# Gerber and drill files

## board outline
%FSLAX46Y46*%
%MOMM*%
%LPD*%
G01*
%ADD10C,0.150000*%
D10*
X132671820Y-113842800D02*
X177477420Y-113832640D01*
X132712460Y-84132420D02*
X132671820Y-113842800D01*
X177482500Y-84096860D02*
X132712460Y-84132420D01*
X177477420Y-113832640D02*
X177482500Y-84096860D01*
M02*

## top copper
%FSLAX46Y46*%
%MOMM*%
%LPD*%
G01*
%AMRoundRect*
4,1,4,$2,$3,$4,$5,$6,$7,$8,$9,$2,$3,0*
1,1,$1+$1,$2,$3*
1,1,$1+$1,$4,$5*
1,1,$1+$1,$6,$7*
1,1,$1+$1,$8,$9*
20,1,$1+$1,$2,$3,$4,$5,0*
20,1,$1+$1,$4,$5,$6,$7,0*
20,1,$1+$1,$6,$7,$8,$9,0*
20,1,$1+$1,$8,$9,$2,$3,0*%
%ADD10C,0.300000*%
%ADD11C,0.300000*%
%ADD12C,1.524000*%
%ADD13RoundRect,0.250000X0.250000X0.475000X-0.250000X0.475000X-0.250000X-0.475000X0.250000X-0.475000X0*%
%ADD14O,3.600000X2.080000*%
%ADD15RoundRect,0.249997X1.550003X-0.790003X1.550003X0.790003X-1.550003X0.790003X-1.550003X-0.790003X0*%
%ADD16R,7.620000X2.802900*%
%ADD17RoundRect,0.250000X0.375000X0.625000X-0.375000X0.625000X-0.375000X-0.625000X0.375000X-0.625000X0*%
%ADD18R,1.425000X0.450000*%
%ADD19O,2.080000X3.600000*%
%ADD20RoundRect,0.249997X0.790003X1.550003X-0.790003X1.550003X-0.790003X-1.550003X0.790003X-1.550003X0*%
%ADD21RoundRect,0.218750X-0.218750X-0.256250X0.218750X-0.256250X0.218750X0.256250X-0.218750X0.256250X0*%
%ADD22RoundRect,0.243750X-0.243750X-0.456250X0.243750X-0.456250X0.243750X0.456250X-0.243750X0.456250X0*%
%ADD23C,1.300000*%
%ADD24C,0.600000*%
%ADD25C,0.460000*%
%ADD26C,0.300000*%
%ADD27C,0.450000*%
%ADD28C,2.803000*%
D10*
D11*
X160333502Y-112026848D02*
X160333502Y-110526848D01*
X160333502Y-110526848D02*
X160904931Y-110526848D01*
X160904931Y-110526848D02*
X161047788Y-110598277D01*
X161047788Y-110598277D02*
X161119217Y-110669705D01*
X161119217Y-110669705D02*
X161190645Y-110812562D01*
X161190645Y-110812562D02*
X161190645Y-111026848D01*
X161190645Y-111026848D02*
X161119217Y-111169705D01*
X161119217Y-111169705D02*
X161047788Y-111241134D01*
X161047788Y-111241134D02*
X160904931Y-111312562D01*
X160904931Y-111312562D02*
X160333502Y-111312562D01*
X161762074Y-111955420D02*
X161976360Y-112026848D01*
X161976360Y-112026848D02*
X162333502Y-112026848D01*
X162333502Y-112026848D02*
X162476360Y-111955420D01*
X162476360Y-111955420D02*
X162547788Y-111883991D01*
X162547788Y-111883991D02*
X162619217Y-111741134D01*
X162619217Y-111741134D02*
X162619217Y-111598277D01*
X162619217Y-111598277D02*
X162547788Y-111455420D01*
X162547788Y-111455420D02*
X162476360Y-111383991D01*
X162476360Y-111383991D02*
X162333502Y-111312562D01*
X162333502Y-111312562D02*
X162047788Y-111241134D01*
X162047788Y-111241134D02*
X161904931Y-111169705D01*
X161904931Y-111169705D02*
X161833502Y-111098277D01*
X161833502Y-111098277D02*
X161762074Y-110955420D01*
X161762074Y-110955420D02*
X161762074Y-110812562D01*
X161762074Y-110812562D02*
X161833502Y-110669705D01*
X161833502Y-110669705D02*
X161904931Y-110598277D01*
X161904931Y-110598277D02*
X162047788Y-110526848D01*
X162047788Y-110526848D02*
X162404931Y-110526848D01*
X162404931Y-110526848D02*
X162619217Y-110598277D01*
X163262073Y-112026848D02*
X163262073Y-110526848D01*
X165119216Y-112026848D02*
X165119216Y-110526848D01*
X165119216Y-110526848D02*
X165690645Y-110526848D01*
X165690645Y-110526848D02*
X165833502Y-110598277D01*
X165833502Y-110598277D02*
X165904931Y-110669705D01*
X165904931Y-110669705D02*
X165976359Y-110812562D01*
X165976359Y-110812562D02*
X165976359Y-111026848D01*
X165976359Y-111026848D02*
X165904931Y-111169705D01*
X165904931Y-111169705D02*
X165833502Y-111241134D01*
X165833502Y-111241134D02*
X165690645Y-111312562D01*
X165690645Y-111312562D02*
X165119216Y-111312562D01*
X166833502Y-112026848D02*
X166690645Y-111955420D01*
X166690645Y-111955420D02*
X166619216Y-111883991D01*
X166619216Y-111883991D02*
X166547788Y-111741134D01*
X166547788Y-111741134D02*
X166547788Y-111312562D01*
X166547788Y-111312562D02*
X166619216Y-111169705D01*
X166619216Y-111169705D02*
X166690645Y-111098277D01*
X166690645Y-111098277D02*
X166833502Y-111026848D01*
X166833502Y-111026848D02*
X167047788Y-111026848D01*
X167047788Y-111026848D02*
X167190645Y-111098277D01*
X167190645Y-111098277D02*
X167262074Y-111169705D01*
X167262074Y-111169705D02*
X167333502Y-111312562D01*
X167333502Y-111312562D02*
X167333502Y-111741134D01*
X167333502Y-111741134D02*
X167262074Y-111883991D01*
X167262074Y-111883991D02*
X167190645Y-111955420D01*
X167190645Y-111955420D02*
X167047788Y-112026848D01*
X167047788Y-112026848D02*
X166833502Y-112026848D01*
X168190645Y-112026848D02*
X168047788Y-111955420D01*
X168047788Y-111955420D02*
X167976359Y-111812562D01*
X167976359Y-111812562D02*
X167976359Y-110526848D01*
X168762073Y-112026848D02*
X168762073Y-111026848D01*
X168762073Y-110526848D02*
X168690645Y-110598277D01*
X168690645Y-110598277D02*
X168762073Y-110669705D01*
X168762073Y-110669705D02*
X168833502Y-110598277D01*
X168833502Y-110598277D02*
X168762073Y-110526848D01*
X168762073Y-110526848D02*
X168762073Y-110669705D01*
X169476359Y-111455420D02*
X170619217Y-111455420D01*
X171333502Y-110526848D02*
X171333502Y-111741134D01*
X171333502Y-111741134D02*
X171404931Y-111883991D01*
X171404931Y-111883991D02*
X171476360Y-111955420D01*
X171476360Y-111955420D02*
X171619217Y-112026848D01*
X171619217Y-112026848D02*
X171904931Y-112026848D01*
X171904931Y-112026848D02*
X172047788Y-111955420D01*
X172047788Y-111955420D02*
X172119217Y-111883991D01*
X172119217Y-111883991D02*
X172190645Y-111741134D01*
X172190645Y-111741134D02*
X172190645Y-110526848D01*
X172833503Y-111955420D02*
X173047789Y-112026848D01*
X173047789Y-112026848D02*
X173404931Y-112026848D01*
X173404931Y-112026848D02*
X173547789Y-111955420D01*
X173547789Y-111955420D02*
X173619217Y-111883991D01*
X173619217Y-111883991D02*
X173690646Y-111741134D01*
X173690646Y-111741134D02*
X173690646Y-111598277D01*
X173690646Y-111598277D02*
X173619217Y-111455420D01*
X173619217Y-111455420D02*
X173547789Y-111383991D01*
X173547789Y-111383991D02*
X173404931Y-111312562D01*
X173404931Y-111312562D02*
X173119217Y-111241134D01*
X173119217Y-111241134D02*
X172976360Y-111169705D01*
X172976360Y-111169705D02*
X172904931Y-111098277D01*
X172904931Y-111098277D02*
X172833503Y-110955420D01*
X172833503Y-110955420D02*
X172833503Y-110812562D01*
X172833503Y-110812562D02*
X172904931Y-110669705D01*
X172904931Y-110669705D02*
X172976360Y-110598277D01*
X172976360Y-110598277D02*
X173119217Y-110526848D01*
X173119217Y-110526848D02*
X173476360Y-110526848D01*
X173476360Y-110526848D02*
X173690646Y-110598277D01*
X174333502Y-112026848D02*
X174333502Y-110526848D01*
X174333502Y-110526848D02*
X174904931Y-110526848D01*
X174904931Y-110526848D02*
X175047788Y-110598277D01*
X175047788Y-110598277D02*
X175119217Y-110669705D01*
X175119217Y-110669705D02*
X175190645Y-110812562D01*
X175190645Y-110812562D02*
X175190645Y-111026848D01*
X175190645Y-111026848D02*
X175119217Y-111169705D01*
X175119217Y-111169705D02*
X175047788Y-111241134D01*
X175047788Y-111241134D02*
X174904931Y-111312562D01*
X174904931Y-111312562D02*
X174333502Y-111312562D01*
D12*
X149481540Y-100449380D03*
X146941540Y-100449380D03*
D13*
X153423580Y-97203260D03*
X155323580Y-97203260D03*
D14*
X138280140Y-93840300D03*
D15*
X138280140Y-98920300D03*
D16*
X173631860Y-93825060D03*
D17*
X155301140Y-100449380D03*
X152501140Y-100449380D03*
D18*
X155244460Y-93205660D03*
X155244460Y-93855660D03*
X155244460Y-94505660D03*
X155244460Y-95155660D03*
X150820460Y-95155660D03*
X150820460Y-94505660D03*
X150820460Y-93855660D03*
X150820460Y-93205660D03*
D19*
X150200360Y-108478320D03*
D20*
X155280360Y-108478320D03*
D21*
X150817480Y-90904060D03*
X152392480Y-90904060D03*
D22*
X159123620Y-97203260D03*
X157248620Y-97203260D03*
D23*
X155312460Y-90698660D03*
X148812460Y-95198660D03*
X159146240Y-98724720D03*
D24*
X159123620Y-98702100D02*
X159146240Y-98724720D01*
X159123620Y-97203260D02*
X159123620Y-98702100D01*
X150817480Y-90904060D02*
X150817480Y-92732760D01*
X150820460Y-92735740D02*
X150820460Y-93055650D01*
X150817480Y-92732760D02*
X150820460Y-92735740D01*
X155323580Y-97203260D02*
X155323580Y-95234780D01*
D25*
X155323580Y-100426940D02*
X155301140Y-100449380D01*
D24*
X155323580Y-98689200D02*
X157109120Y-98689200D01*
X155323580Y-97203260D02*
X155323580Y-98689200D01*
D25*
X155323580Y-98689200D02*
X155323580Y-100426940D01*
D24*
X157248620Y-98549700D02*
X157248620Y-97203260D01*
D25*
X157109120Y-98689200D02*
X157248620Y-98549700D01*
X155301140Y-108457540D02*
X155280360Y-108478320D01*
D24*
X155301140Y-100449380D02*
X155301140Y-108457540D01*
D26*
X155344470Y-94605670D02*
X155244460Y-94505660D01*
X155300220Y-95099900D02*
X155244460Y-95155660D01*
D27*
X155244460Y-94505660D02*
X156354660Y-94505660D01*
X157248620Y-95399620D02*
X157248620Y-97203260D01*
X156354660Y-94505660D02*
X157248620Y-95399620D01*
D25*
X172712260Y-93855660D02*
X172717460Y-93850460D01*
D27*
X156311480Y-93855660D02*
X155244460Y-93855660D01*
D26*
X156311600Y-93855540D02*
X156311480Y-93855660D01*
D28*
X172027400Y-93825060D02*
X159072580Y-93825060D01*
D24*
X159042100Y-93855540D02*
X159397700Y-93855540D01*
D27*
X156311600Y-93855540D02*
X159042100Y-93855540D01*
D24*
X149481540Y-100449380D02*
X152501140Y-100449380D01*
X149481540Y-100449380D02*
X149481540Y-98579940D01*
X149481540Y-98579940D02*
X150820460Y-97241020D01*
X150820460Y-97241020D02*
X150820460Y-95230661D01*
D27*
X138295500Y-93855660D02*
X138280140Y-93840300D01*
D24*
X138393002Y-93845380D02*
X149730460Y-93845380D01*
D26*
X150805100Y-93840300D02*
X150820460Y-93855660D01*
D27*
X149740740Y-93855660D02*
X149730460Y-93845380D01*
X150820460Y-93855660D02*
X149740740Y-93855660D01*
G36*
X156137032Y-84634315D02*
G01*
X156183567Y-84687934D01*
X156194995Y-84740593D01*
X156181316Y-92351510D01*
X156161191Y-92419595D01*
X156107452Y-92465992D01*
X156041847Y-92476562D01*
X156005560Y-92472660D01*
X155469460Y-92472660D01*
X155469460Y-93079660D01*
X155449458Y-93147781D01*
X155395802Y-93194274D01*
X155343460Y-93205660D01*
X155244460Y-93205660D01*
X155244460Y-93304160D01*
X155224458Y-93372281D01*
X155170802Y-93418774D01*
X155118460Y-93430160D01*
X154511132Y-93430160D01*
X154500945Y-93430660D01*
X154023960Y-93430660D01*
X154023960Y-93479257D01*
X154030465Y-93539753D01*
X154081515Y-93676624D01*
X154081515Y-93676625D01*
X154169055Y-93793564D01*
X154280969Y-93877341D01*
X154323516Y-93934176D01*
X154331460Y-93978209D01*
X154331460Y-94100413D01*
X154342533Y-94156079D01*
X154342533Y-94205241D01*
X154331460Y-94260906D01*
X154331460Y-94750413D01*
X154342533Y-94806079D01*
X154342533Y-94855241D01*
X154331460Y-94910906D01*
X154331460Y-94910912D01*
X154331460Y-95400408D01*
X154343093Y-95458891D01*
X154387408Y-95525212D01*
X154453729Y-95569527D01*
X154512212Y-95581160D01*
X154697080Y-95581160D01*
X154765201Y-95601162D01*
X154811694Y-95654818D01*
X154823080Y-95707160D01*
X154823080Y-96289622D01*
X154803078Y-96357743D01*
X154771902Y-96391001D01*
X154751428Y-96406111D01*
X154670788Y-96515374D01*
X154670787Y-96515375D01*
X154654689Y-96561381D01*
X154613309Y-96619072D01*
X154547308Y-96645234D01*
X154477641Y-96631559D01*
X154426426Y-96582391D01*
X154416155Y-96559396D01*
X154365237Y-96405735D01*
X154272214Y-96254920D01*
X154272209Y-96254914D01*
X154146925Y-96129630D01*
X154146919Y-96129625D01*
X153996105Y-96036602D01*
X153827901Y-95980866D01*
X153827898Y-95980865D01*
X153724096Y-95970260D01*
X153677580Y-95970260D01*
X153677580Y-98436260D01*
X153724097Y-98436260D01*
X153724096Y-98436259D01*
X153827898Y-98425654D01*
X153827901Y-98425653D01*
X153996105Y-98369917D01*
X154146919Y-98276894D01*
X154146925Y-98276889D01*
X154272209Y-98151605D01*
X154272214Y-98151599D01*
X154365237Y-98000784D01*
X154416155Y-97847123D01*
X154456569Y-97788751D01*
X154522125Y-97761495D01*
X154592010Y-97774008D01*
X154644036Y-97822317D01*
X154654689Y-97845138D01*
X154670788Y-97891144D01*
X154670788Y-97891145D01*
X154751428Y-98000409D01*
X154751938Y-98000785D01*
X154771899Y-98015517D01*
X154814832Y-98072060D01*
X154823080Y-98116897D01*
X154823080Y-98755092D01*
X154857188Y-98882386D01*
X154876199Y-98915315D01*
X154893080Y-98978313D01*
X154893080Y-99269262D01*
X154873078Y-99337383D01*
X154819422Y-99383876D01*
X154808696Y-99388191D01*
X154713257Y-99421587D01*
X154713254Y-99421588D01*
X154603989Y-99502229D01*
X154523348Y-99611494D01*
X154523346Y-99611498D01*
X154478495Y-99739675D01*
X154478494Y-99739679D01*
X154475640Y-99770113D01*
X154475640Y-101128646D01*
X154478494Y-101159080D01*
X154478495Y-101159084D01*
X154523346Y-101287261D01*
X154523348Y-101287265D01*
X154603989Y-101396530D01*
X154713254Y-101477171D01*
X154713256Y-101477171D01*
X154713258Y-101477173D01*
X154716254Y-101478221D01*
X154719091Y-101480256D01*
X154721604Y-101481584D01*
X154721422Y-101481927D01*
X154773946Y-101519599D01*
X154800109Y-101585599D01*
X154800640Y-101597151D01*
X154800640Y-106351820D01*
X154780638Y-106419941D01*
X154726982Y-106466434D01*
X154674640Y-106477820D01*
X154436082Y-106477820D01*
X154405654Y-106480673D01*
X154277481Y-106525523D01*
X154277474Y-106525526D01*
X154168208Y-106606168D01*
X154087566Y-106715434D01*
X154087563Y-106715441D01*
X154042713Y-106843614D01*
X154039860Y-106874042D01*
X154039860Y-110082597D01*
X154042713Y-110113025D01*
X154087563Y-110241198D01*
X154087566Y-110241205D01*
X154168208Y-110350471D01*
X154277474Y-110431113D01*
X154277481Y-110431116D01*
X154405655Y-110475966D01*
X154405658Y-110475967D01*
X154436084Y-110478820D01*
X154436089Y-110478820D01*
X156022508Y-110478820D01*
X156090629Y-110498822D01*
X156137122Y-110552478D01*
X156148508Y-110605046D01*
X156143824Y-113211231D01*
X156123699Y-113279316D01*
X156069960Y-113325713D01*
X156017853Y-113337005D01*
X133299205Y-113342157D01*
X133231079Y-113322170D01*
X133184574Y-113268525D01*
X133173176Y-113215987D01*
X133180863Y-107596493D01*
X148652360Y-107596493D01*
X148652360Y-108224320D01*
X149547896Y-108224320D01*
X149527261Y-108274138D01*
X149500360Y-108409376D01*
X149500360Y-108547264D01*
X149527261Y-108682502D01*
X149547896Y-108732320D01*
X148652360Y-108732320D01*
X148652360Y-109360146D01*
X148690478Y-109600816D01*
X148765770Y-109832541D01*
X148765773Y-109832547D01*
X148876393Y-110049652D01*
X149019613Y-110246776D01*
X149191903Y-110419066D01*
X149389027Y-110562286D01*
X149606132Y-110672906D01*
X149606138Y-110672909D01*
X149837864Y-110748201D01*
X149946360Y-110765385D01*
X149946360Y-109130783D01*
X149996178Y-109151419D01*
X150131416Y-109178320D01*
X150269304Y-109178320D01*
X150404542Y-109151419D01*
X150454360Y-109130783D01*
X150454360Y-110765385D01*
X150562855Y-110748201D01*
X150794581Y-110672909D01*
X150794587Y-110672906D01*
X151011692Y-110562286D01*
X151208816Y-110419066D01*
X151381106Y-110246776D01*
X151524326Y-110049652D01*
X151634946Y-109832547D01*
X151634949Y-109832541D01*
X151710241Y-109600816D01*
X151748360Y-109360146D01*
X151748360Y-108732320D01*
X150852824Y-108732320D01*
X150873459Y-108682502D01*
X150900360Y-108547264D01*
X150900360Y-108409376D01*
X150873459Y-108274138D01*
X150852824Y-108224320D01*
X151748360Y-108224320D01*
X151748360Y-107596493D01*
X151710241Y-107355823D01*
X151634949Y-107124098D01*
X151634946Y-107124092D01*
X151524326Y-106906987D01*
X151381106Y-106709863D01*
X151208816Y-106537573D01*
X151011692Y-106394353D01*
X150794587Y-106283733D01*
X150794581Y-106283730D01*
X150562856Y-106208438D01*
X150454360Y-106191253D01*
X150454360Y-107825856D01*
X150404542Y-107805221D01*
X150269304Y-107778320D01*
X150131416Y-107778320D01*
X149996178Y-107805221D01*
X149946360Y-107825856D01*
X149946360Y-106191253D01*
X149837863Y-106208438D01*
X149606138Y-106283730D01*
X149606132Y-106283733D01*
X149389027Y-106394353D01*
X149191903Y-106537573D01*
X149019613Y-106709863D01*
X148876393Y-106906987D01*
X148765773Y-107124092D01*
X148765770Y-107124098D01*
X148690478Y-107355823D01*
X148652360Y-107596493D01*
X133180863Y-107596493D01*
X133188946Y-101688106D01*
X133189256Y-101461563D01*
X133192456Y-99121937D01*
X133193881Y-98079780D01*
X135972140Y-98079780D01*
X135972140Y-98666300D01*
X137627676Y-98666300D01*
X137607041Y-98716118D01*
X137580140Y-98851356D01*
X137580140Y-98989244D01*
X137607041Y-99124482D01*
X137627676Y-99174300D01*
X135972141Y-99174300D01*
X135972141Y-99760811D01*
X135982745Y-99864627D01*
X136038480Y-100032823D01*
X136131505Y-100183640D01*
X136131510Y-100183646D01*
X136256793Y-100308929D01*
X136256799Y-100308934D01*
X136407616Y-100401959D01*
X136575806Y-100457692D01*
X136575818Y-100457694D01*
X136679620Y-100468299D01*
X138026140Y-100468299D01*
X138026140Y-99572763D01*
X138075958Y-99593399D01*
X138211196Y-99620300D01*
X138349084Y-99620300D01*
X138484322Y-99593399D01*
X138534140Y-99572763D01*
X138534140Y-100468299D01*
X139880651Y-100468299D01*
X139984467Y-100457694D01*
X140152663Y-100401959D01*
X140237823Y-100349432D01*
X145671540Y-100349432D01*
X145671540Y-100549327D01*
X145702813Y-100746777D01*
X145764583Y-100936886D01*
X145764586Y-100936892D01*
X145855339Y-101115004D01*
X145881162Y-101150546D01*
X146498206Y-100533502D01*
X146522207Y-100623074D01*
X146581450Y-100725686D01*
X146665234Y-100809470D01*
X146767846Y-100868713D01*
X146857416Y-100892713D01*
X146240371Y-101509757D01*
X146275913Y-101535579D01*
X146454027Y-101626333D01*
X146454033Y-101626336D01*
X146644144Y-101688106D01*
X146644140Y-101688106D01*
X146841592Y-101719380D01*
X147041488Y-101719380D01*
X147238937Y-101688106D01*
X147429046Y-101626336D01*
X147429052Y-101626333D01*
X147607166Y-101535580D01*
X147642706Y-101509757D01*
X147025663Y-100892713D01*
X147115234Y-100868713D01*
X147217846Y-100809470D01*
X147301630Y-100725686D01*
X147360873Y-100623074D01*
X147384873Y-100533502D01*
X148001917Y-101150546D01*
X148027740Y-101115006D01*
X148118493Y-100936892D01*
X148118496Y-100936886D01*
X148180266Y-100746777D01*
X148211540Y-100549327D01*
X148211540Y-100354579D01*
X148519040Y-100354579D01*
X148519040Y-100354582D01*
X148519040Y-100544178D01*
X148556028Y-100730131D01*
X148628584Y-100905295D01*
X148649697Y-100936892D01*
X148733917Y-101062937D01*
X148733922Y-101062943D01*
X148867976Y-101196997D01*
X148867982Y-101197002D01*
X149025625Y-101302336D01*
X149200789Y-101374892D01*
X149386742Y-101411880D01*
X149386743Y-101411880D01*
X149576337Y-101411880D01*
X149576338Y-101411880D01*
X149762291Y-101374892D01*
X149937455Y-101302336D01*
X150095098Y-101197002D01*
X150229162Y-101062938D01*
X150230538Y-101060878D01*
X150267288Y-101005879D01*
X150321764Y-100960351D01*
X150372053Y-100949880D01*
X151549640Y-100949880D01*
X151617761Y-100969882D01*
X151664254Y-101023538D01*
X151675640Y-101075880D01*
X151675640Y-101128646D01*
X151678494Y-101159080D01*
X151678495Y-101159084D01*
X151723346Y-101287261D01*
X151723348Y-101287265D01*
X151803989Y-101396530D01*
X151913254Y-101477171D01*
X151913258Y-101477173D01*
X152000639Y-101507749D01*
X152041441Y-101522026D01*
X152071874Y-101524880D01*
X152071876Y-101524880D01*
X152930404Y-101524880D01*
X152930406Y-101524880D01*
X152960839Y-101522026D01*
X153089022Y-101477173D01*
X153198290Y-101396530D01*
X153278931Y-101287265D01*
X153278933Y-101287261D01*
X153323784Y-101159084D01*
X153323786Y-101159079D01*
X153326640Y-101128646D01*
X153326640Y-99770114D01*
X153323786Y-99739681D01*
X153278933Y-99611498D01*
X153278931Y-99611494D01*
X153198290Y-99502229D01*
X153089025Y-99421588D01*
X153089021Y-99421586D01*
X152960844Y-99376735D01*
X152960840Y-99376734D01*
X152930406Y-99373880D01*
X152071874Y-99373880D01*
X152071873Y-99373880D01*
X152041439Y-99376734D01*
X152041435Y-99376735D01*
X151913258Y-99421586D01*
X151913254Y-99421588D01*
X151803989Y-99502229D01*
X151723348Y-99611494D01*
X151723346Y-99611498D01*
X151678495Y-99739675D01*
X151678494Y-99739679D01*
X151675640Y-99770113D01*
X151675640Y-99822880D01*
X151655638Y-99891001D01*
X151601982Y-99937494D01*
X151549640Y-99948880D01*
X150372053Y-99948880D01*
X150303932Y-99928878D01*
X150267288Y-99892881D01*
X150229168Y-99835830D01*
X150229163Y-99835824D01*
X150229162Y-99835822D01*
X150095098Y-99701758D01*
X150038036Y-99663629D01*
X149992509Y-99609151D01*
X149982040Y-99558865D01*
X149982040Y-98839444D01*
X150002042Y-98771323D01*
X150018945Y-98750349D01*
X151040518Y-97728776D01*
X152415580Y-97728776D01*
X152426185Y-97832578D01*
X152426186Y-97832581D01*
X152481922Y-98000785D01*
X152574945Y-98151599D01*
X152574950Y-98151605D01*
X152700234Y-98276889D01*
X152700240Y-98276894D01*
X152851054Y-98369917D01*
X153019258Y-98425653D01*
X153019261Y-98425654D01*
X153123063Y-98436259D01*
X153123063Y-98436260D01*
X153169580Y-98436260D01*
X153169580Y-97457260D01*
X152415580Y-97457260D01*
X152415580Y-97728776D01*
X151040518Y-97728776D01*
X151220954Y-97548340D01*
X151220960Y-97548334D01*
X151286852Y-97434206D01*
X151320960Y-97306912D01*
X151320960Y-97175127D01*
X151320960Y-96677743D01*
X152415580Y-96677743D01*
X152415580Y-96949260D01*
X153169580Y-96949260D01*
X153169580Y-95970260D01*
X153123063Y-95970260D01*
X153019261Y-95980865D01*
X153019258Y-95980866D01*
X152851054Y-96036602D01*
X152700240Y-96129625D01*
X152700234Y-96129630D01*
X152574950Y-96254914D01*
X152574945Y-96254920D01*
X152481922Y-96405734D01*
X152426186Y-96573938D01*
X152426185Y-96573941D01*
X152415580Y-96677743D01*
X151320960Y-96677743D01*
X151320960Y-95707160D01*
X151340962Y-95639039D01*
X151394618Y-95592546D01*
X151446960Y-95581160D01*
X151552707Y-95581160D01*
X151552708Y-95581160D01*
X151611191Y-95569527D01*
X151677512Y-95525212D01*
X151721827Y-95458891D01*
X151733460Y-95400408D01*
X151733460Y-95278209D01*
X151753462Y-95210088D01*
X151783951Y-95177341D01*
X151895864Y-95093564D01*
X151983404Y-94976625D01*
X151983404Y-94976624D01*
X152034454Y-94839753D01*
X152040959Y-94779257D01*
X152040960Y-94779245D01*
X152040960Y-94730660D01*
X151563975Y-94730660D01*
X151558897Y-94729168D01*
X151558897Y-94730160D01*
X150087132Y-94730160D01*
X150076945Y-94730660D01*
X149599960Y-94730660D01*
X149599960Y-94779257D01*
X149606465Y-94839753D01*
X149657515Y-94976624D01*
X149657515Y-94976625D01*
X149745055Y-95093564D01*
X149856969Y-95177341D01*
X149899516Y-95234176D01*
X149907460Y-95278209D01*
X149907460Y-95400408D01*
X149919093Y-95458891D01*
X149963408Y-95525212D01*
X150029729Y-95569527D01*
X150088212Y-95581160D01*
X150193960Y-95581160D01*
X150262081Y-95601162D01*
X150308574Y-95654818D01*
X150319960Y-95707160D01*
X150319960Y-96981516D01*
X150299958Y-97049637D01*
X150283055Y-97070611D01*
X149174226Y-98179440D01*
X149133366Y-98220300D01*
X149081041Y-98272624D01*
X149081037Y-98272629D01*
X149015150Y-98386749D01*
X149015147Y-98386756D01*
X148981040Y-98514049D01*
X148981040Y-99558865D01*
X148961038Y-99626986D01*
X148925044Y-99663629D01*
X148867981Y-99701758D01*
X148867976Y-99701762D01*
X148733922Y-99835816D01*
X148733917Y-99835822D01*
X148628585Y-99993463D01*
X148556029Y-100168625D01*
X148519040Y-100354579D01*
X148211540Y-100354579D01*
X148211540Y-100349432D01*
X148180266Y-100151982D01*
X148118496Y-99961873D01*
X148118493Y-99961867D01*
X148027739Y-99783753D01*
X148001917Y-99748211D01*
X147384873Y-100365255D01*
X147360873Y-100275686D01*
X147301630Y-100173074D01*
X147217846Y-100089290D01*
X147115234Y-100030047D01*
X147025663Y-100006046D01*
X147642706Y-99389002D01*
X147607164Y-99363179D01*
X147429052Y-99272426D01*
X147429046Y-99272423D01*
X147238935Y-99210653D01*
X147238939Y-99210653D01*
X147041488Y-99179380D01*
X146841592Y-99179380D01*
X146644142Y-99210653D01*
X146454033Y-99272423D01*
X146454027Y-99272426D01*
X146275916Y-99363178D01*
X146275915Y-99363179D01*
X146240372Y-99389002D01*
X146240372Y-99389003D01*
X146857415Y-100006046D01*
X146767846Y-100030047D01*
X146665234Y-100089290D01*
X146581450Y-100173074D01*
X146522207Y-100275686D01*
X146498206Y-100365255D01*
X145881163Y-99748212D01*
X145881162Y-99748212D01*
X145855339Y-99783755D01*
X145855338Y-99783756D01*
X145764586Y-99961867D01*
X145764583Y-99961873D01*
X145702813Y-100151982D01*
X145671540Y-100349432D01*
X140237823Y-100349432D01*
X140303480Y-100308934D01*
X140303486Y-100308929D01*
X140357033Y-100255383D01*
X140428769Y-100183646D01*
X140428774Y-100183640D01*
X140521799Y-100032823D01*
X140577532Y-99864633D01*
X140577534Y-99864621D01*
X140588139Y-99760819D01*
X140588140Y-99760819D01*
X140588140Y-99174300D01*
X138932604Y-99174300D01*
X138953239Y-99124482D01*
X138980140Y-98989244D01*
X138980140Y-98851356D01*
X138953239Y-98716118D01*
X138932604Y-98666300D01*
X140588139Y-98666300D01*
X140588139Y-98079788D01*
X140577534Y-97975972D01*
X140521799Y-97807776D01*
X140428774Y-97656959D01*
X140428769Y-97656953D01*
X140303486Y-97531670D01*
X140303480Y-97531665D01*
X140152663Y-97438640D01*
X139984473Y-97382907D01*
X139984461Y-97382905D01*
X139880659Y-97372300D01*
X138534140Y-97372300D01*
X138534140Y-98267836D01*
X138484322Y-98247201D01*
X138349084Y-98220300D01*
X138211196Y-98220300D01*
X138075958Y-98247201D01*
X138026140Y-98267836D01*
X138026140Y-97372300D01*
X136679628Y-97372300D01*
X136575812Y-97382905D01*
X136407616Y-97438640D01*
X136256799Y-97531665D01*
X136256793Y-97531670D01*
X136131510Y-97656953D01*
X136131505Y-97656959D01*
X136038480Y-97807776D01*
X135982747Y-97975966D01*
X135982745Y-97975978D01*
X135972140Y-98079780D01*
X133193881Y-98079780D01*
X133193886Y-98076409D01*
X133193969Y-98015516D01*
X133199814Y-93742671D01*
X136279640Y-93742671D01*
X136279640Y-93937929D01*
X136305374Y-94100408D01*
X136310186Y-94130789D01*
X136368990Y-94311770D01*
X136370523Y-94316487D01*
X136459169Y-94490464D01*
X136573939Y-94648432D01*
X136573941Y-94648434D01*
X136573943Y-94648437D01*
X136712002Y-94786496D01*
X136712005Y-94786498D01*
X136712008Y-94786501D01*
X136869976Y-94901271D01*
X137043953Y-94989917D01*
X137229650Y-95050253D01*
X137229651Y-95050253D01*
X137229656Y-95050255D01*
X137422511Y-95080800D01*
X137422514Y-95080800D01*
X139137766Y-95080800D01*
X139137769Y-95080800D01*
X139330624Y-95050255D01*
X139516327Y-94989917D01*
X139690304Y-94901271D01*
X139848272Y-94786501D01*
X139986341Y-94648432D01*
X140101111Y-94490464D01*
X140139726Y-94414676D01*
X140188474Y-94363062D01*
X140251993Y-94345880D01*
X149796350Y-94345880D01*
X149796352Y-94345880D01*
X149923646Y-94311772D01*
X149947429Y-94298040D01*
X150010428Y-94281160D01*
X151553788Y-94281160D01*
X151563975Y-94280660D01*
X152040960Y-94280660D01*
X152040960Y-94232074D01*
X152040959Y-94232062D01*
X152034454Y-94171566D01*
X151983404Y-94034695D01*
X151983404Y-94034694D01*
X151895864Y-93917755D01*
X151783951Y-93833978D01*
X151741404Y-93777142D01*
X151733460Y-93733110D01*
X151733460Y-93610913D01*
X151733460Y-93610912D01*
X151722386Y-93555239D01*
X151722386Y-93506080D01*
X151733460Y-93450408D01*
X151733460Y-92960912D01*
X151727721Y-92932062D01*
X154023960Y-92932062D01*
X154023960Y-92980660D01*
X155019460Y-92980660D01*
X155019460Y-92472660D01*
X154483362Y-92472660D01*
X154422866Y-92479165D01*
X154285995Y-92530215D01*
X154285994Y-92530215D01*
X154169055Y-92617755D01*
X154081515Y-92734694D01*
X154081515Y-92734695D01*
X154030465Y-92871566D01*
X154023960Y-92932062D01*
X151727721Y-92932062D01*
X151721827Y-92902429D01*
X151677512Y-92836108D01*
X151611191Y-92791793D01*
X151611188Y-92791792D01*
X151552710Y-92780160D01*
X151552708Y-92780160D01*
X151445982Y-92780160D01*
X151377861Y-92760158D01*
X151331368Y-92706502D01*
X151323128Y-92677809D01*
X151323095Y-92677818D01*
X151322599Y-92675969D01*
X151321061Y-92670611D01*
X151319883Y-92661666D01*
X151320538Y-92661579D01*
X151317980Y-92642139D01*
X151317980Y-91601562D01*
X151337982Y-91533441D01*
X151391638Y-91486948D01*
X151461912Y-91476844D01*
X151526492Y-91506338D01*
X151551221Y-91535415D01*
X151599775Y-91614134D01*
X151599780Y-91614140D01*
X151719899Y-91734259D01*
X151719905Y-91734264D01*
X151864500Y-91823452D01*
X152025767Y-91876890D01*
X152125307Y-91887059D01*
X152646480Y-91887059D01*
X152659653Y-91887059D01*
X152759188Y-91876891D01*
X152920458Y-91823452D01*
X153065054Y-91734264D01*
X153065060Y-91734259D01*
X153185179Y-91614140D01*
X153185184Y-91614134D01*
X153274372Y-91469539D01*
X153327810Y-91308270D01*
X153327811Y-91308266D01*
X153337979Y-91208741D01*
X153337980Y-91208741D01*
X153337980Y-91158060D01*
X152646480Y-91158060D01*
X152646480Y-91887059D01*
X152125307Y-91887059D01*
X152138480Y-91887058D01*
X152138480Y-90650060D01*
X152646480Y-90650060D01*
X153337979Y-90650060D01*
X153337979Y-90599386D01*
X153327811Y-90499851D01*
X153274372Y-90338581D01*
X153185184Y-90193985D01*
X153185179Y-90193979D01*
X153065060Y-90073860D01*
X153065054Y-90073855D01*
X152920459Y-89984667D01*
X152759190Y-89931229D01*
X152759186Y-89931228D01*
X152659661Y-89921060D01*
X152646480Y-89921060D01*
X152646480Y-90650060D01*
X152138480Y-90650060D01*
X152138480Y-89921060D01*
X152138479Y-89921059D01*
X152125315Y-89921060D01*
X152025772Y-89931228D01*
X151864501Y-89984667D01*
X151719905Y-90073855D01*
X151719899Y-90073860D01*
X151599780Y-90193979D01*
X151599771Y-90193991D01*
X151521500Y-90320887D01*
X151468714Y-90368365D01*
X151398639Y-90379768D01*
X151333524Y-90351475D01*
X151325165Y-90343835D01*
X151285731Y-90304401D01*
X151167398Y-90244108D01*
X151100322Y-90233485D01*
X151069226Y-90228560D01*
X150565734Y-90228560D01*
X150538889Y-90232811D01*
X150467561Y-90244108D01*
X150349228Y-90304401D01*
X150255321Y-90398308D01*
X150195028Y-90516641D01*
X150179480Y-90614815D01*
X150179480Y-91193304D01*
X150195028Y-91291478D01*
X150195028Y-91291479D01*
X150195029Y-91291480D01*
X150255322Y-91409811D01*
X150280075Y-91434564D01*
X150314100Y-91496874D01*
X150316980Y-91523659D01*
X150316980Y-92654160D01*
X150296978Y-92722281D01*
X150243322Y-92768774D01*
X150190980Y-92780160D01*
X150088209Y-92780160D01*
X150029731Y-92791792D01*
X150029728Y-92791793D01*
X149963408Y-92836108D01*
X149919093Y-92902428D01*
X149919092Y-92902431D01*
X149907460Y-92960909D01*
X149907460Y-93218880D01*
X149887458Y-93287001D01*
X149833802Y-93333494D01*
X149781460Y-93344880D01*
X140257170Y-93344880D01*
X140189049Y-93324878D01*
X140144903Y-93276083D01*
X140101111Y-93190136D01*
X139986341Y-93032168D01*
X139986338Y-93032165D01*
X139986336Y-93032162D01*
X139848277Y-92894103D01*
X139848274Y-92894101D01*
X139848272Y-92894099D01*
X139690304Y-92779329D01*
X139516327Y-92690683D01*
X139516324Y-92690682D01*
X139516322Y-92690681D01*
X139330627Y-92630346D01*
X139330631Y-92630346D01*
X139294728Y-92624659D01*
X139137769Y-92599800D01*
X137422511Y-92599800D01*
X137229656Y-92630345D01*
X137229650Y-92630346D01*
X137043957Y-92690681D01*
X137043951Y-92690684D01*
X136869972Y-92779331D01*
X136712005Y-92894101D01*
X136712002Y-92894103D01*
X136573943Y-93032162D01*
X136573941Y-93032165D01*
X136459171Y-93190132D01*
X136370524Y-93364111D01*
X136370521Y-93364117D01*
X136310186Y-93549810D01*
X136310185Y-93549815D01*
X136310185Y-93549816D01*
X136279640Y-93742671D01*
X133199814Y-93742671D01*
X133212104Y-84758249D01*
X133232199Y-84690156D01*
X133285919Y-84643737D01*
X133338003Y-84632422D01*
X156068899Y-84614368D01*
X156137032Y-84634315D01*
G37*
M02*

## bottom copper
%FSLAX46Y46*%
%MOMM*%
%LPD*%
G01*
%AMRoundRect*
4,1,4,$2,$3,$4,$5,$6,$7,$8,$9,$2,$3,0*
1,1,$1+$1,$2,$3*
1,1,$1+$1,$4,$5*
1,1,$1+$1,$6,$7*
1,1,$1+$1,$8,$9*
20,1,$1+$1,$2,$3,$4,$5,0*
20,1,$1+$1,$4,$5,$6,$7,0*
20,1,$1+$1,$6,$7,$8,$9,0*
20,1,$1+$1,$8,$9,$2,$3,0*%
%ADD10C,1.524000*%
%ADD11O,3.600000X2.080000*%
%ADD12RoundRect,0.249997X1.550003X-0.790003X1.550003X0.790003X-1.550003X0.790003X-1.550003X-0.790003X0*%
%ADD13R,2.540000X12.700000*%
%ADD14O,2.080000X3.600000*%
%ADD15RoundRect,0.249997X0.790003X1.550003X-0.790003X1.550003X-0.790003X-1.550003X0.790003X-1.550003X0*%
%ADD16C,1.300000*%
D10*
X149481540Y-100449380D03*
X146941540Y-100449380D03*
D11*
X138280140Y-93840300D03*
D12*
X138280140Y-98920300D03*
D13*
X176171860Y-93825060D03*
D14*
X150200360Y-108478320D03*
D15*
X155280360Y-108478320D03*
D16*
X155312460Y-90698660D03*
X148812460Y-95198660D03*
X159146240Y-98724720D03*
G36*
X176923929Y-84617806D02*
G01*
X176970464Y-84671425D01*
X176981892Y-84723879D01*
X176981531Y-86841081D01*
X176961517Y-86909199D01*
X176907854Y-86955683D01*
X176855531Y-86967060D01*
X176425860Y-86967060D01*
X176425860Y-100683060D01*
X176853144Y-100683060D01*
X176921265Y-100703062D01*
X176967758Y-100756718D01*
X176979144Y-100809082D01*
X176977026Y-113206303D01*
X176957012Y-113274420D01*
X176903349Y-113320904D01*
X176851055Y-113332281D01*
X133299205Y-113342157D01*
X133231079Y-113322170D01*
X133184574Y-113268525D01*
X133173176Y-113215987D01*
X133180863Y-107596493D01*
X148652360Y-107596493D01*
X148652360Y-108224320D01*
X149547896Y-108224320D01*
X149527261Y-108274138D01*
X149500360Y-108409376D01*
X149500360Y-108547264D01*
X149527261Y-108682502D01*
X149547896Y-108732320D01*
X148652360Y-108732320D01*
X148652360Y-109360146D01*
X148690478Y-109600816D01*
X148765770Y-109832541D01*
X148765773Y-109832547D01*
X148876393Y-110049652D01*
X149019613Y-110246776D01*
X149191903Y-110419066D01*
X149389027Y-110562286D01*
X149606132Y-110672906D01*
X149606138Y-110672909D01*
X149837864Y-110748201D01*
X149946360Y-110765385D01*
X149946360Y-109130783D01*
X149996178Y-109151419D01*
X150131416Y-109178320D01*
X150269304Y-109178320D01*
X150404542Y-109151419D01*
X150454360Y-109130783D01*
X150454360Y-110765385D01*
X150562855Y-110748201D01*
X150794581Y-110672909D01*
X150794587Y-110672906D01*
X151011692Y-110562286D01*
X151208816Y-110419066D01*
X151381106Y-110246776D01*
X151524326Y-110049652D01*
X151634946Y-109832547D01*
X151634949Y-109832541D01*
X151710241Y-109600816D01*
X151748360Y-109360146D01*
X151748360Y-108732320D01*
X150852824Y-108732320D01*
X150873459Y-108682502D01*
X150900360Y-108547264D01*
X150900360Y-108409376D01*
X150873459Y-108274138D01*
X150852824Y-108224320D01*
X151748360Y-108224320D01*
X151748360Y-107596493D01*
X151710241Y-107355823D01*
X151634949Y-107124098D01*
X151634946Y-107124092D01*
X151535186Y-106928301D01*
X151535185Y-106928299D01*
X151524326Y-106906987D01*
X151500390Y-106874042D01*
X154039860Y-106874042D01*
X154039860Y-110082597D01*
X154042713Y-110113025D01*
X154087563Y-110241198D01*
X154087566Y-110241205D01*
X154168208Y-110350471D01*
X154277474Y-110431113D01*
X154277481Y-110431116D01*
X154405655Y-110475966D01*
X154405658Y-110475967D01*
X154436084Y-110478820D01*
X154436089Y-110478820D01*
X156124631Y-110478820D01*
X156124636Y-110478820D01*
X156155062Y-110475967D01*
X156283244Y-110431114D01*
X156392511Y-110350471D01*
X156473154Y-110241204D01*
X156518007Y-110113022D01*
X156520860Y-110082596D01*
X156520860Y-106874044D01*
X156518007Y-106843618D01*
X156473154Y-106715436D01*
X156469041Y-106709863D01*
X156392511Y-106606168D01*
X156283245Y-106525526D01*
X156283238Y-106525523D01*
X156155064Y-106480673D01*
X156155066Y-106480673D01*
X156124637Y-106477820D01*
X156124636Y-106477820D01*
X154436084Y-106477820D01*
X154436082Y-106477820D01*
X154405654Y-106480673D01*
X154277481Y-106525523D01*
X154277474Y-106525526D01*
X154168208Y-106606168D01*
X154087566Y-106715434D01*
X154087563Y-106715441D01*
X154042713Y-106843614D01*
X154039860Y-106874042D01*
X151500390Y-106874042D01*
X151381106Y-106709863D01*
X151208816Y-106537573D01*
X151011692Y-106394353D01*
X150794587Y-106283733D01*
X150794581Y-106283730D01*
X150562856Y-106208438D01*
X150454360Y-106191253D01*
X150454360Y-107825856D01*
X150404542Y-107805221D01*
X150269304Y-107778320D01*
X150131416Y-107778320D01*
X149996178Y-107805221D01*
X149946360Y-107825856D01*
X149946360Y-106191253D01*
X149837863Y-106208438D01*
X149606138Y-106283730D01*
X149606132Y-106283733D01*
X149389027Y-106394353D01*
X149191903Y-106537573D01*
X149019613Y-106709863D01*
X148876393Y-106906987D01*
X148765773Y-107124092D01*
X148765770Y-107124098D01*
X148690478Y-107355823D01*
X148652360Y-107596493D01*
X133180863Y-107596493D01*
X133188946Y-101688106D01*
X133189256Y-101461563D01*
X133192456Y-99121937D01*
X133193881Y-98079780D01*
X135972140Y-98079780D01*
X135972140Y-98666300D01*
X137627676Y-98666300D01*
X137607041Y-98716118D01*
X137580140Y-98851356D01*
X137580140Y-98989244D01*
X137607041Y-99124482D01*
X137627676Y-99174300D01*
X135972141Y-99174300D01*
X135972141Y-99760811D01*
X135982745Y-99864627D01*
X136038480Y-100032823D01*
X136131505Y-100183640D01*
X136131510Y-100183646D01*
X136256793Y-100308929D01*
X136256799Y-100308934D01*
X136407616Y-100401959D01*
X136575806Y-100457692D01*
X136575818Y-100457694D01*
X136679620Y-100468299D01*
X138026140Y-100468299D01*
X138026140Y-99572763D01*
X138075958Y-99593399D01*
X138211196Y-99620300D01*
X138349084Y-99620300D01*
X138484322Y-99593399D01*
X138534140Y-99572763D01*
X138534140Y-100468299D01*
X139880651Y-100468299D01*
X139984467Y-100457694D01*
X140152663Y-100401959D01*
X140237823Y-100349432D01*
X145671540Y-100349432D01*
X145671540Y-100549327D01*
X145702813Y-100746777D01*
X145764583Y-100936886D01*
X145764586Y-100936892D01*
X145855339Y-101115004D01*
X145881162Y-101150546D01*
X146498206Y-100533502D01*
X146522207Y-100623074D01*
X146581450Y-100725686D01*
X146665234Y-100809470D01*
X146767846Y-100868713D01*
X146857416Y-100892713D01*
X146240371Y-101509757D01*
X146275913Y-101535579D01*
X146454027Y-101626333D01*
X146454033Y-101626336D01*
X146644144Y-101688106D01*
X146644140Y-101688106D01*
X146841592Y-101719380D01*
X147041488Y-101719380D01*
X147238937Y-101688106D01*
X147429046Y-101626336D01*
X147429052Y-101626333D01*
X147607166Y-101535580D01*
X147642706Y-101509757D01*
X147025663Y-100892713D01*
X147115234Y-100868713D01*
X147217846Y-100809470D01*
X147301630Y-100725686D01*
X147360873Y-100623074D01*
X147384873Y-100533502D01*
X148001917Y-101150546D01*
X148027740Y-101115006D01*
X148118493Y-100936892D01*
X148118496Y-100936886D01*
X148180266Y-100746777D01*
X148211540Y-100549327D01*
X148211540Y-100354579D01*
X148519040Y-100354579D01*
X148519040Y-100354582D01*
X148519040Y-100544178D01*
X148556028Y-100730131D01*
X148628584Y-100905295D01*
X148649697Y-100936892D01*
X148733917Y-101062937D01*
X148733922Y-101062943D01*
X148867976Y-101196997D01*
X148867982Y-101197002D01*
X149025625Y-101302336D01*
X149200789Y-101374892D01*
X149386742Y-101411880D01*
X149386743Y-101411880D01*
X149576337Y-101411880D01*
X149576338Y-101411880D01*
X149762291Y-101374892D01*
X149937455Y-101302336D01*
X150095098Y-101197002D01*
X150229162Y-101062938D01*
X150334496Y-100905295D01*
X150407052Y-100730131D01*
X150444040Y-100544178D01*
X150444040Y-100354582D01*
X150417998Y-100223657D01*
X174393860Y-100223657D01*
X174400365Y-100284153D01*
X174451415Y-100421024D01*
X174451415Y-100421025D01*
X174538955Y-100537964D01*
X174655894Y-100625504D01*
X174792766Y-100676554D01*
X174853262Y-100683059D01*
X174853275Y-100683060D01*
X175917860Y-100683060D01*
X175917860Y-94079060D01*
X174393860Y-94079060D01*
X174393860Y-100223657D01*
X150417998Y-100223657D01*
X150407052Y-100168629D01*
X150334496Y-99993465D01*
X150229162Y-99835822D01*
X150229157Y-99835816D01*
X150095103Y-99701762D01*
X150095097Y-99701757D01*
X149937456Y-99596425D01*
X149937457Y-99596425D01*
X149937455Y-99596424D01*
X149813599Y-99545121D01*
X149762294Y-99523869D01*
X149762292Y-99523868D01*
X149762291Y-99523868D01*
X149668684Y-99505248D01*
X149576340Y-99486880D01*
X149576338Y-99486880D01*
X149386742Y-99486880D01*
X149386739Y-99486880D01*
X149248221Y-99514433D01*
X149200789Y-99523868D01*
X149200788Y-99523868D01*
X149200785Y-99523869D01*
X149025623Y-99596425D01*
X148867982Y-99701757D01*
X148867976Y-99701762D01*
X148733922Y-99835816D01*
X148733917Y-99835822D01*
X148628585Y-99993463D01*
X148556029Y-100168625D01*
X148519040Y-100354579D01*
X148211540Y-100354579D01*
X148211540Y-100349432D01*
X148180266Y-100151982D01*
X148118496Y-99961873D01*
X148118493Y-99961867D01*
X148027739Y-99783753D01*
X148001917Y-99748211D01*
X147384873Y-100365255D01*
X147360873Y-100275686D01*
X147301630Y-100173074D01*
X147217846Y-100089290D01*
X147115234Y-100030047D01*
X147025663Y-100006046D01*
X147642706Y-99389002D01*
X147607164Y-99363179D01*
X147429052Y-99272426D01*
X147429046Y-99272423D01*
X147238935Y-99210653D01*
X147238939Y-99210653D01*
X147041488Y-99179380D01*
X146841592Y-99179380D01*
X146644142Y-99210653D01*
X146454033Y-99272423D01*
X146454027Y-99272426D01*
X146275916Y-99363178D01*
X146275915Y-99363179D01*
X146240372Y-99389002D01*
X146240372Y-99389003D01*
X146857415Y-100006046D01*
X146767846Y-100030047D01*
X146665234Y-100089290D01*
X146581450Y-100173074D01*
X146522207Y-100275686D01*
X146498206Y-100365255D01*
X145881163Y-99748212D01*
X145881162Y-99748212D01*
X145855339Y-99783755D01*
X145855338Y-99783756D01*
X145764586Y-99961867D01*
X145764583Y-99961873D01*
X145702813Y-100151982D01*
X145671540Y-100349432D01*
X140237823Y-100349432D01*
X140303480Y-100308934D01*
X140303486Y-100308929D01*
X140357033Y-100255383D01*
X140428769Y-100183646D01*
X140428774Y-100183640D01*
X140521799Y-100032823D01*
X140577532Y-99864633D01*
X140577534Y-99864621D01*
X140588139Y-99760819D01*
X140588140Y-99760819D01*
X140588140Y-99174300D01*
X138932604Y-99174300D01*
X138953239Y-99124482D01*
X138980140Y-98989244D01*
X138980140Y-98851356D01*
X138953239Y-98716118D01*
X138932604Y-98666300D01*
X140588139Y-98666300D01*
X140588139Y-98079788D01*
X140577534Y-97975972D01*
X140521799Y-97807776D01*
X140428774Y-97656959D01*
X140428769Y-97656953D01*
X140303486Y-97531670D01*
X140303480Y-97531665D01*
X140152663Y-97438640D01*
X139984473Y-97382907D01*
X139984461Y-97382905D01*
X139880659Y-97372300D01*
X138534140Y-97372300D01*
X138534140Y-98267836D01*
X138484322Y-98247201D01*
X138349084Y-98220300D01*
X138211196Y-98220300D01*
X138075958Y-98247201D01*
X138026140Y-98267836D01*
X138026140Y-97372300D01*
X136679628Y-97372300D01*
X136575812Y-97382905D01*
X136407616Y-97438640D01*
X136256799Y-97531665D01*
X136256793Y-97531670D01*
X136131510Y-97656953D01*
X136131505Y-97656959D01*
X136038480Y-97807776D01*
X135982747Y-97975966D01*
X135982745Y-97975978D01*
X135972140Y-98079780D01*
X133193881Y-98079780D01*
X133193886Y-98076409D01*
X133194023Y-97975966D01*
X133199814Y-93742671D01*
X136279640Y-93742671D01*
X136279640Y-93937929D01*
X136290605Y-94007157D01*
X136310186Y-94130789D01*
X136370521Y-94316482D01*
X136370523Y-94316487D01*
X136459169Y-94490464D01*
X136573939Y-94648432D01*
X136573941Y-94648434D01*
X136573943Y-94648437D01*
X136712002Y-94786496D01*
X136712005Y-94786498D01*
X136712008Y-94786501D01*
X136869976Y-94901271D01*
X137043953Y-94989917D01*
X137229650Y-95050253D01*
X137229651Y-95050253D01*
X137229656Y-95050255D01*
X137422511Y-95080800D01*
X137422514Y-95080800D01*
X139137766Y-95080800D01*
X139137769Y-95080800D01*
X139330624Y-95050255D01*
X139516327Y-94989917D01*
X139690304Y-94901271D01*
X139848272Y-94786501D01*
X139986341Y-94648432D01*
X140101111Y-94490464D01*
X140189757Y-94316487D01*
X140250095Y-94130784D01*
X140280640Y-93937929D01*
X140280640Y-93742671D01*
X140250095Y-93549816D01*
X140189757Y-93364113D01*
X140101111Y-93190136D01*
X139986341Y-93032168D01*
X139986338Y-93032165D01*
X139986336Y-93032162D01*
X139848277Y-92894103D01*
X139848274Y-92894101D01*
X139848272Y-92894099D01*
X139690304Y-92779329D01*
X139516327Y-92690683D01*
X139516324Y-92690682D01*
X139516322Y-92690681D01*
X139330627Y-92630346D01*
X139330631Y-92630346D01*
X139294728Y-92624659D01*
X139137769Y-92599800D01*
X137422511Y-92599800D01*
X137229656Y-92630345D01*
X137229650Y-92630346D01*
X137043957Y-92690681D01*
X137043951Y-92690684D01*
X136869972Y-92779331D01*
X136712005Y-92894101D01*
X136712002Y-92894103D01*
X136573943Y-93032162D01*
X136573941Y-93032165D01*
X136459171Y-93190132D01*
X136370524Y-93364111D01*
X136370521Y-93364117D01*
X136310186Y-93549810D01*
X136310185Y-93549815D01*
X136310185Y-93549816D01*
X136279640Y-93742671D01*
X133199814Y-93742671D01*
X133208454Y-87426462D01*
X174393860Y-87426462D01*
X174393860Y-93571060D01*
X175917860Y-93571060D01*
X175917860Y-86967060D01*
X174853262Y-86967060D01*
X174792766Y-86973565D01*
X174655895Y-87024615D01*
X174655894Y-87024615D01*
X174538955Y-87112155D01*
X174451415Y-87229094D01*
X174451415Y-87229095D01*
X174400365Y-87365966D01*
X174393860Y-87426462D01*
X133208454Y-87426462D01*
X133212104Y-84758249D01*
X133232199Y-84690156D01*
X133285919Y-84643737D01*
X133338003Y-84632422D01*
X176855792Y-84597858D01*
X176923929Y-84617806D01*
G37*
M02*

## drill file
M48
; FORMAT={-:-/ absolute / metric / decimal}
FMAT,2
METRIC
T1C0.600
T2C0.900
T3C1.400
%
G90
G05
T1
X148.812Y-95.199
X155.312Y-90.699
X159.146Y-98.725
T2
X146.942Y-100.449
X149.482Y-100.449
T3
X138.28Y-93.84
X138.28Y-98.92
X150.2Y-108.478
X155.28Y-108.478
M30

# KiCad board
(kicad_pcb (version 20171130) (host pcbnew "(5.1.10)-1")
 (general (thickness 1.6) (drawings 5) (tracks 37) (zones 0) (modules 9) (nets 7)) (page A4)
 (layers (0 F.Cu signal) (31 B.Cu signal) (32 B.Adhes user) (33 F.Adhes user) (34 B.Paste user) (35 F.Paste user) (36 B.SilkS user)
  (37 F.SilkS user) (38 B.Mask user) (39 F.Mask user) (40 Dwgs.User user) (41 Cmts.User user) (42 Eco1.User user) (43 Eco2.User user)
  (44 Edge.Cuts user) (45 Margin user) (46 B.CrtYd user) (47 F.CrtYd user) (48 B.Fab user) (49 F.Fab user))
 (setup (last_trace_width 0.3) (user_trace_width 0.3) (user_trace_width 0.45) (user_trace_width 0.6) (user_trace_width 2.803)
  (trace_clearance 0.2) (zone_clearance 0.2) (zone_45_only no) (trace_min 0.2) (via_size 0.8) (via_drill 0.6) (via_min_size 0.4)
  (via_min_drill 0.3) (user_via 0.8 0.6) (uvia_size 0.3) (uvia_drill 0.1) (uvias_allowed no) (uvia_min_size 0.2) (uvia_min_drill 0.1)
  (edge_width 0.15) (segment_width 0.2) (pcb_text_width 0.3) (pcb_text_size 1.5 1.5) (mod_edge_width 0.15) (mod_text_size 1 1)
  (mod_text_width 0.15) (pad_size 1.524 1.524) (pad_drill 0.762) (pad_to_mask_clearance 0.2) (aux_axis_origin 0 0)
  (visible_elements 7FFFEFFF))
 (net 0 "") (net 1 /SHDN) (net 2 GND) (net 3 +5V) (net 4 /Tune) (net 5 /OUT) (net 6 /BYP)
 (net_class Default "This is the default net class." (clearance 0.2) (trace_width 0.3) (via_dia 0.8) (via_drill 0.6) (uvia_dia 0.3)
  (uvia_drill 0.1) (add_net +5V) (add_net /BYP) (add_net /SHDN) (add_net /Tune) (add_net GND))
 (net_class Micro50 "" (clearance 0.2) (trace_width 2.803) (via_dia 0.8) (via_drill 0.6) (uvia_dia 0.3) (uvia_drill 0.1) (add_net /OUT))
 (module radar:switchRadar (layer F.Cu) (at 146.94154 100.44938)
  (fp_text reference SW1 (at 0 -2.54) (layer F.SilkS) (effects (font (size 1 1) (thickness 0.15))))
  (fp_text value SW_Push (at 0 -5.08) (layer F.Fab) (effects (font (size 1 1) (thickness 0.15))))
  (pad 2 thru_hole circle (at 2.54 0) (size 1.524 1.524) (drill 0.9) (layers *.Cu *.Mask) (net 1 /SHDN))
  (pad 1 thru_hole circle (at 0 0) (size 1.524 1.524) (drill 0.9) (layers *.Cu *.Mask) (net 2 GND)))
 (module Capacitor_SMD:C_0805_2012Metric (layer F.Cu) (at 154.37358 97.20326 180)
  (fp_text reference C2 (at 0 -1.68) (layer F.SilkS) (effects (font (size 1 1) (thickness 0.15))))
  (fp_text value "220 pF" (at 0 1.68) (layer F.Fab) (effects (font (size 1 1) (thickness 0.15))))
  (pad 2 smd roundrect (at 0.95 0 180) (size 1 1.45) (layers F.Cu F.Paste F.Mask) (roundrect_rratio 0.25) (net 2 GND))
  (pad 1 smd roundrect (at -0.95 0 180) (size 1 1.45) (layers F.Cu F.Paste F.Mask) (roundrect_rratio 0.25) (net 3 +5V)))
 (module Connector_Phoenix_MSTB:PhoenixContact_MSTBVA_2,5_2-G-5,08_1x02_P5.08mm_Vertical (layer F.Cu) (at 138.28014 98.9203 90)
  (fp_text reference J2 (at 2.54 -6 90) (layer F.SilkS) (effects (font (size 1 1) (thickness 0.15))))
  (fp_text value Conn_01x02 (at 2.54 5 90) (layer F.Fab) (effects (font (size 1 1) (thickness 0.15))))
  (pad 2 thru_hole oval (at 5.08 0 90) (size 2.08 3.6) (drill 1.4) (layers *.Cu *.Mask) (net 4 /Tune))
  (pad 1 thru_hole roundrect (at 0 0 90) (size 2.08 3.6) (drill 1.4) (layers *.Cu *.Mask) (roundrect_rratio 0.1201908653846154) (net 2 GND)))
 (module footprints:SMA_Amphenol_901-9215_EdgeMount (layer F.Cu) (at 172.36186 93.82506)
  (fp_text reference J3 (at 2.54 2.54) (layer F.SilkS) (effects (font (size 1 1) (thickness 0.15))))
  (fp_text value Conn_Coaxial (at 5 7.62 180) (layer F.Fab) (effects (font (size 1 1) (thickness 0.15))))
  (pad 1 smd rect (at 1.27 0 90) (size 2.8029 7.62) (layers F.Cu F.Paste F.Mask) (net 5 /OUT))
  (pad 2 smd rect (at 3.81 0 180) (size 2.54 12.7) (layers B.Cu B.Paste B.Mask) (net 2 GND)))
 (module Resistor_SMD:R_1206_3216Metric (layer F.Cu) (at 153.90114 100.44938 180)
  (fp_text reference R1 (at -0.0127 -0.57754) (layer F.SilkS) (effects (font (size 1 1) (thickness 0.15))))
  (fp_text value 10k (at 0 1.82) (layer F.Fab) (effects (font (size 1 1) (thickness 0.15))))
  (pad 1 smd roundrect (at -1.4 0 180) (size 1.25 1.75) (layers F.Cu F.Paste F.Mask) (roundrect_rratio 0.2) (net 3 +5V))
  (pad 2 smd roundrect (at 1.4 0 180) (size 1.25 1.75) (layers F.Cu F.Paste F.Mask) (roundrect_rratio 0.2) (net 1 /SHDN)))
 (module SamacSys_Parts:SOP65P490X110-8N (layer F.Cu) (at 153.03246 94.18066)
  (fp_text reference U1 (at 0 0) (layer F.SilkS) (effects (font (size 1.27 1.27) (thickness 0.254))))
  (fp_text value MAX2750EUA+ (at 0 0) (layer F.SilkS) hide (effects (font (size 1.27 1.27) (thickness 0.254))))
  (pad 8 smd rect (at 2.212 -0.975 90) (size 0.45 1.425) (layers F.Cu F.Paste F.Mask) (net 2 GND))
  (pad 7 smd rect (at 2.212 -0.325 90) (size 0.45 1.425) (layers F.Cu F.Paste F.Mask) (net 5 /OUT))
  (pad 6 smd rect (at 2.212 0.325 90) (size 0.45 1.425) (layers F.Cu F.Paste F.Mask) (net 3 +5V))
  (pad 5 smd rect (at 2.212 0.975 90) (size 0.45 1.425) (layers F.Cu F.Paste F.Mask) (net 3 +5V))
  (pad 4 smd rect (at -2.212 0.975 90) (size 0.45 1.425) (layers F.Cu F.Paste F.Mask) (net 1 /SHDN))
  (pad 3 smd rect (at -2.212 0.325 90) (size 0.45 1.425) (layers F.Cu F.Paste F.Mask) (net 2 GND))
  (pad 2 smd rect (at -2.212 -0.325 90) (size 0.45 1.425) (layers F.Cu F.Paste F.Mask) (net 4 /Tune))
  (pad 1 smd rect (at -2.212 -0.975 90) (size 0.45 1.425) (layers F.Cu F.Paste F.Mask) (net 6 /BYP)))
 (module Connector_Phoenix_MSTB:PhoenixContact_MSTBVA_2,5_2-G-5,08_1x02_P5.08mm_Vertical (layer F.Cu) (at 155.28036 108.47832 180)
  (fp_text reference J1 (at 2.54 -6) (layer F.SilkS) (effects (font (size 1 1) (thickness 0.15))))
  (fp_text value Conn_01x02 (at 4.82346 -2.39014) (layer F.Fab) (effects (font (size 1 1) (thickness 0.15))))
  (pad 2 thru_hole oval (at 5.08 0 180) (size 2.08 3.6) (drill 1.4) (layers *.Cu *.Mask) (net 2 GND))
  (pad 1 thru_hole roundrect (at 0 0 180) (size 2.08 3.6) (drill 1.4) (layers *.Cu *.Mask) (roundrect_rratio 0.1201908653846154) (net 3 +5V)))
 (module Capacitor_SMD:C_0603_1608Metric (layer F.Cu) (at 151.60498 90.90406)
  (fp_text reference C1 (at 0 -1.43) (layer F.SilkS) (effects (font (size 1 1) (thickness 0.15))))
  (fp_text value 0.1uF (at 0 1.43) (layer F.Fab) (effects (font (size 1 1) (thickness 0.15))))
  (pad 1 smd roundrect (at -0.7875 0) (size 0.875 0.95) (layers F.Cu F.Paste F.Mask) (roundrect_rratio 0.25) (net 6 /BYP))
  (pad 2 smd roundrect (at 0.7875 0) (size 0.875 0.95) (layers F.Cu F.Paste F.Mask) (roundrect_rratio 0.25) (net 2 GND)))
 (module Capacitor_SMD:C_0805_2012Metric (layer F.Cu) (at 158.18612 97.20326)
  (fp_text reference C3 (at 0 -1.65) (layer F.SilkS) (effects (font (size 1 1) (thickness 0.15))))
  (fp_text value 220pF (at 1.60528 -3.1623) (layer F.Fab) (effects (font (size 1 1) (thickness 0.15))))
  (pad 2 smd roundrect (at 0.9375 0) (size 0.975 1.4) (layers F.Cu F.Paste F.Mask) (roundrect_rratio 0.25) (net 2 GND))
  (pad 1 smd roundrect (at -0.9375 0) (size 0.975 1.4) (layers F.Cu F.Paste F.Mask) (roundrect_rratio 0.25) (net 3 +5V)))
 (gr_line (start 132.67182 113.8428) (end 177.47742 113.83264) (layer Edge.Cuts) (width 0.15))
 (gr_line (start 132.71246 84.13242) (end 132.67182 113.8428) (layer Edge.Cuts) (width 0.15))
 (gr_line (start 177.4825 84.09686) (end 132.71246 84.13242) (layer Edge.Cuts) (width 0.15))
 (gr_line (start 177.47742 113.83264) (end 177.4825 84.09686) (layer Edge.Cuts) (width 0.15))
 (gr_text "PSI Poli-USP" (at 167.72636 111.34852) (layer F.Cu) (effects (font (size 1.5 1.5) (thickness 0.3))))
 (via (at 155.31246 90.69866) (size 1.3) (drill 0.6) (layers F.Cu B.Cu) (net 2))
 (via (at 148.81246 95.19866) (size 1.3) (drill 0.6) (layers F.Cu B.Cu) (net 2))
 (via (at 159.14624 98.72472) (size 1.3) (drill 0.6) (layers F.Cu B.Cu) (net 2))
 (segment (start 159.12362 98.7021) (end 159.14624 98.72472) (width 0.6) (layer F.Cu) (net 2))
 (segment (start 159.12362 97.20326) (end 159.12362 98.7021) (width 0.6) (layer F.Cu) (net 2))
 (segment (start 150.81748 90.90406) (end 150.81748 92.73276) (width 0.6) (layer F.Cu) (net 6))
 (segment (start 150.82046 92.73574) (end 150.82046 93.05565) (width 0.6) (layer F.Cu) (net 6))
 (segment (start 150.81748 92.73276) (end 150.82046 92.73574) (width 0.6) (layer F.Cu) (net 6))
 (segment (start 155.32358 97.20326) (end 155.32358 95.23478) (width 0.6) (layer F.Cu) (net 3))
 (segment (start 155.32358 100.42694) (end 155.30114 100.44938) (width 0.46) (layer F.Cu) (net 3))
 (segment (start 155.32358 98.6892) (end 157.10912 98.6892) (width 0.6) (layer F.Cu) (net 3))
 (segment (start 155.32358 97.20326) (end 155.32358 98.6892) (width 0.6) (layer F.Cu) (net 3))
 (segment (start 155.32358 98.6892) (end 155.32358 100.42694) (width 0.46) (layer F.Cu) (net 3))
 (segment (start 157.24862 98.5497) (end 157.24862 97.20326) (width 0.6) (layer F.Cu) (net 3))
 (segment (start 157.10912 98.6892) (end 157.24862 98.5497) (width 0.46) (layer F.Cu) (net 3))
 (segment (start 155.30114 108.45754) (end 155.28036 108.47832) (width 0.46) (layer F.Cu) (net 3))
 (segment (start 155.30114 100.44938) (end 155.30114 108.45754) (width 0.6) (layer F.Cu) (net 3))
 (segment (start 155.34447 94.60567) (end 155.24446 94.50566) (width 0.3) (layer F.Cu) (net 3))
 (segment (start 155.30022 95.0999) (end 155.24446 95.15566) (width 0.3) (layer F.Cu) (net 3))
 (segment (start 155.24446 94.50566) (end 156.35466 94.50566) (width 0.45) (layer F.Cu) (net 3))
 (segment (start 157.24862 95.39962) (end 157.24862 97.20326) (width 0.45) (layer F.Cu) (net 3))
 (segment (start 156.35466 94.50566) (end 157.24862 95.39962) (width 0.45) (layer F.Cu) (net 3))
 (segment (start 172.71226 93.85566) (end 172.71746 93.85046) (width 0.46) (layer F.Cu) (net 5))
 (segment (start 156.31148 93.85566) (end 155.24446 93.85566) (width 0.45) (layer F.Cu) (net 5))
 (segment (start 156.3116 93.85554) (end 156.31148 93.85566) (width 0.3) (layer F.Cu) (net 5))
 (segment (start 172.0274 93.82506) (end 159.07258 93.82506) (width 2.803) (layer F.Cu) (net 5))
 (segment (start 159.0421 93.85554) (end 159.3977 93.85554) (width 0.6) (layer F.Cu) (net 5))
 (segment (start 156.3116 93.85554) (end 159.0421 93.85554) (width 0.45) (layer F.Cu) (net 5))
 (segment (start 149.48154 100.44938) (end 152.50114 100.44938) (width 0.6) (layer F.Cu) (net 1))
 (segment (start 149.48154 100.44938) (end 149.48154 98.57994) (width 0.6) (layer F.Cu) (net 1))
 (segment (start 149.48154 98.57994) (end 150.82046 97.24102) (width 0.6) (layer F.Cu) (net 1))
 (segment (start 150.82046 97.24102) (end 150.82046 95.230661) (width 0.6) (layer F.Cu) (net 1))
 (segment (start 138.2955 93.85566) (end 138.28014 93.8403) (width 0.45) (layer F.Cu) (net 4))
 (segment (start 138.393002 93.84538) (end 149.73046 93.84538) (width 0.6) (layer F.Cu) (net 4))
 (segment (start 150.8051 93.8403) (end 150.82046 93.85566) (width 0.3) (layer F.Cu) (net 4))
 (segment (start 149.74074 93.85566) (end 149.73046 93.84538) (width 0.45) (layer F.Cu) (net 4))
 (segment (start 150.82046 93.85566) (end 149.74074 93.85566) (width 0.45) (layer F.Cu) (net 4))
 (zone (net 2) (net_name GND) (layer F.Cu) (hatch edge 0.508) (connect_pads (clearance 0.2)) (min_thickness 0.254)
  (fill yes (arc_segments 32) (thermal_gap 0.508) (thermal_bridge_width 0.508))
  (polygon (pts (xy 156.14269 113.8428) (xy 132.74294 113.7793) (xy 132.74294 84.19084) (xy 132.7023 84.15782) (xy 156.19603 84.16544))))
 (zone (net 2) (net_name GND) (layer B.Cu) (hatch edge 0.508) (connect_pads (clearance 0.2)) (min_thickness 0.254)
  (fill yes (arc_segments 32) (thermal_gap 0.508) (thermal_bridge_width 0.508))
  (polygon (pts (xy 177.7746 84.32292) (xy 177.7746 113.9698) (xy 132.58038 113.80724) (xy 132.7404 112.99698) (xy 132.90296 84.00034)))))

